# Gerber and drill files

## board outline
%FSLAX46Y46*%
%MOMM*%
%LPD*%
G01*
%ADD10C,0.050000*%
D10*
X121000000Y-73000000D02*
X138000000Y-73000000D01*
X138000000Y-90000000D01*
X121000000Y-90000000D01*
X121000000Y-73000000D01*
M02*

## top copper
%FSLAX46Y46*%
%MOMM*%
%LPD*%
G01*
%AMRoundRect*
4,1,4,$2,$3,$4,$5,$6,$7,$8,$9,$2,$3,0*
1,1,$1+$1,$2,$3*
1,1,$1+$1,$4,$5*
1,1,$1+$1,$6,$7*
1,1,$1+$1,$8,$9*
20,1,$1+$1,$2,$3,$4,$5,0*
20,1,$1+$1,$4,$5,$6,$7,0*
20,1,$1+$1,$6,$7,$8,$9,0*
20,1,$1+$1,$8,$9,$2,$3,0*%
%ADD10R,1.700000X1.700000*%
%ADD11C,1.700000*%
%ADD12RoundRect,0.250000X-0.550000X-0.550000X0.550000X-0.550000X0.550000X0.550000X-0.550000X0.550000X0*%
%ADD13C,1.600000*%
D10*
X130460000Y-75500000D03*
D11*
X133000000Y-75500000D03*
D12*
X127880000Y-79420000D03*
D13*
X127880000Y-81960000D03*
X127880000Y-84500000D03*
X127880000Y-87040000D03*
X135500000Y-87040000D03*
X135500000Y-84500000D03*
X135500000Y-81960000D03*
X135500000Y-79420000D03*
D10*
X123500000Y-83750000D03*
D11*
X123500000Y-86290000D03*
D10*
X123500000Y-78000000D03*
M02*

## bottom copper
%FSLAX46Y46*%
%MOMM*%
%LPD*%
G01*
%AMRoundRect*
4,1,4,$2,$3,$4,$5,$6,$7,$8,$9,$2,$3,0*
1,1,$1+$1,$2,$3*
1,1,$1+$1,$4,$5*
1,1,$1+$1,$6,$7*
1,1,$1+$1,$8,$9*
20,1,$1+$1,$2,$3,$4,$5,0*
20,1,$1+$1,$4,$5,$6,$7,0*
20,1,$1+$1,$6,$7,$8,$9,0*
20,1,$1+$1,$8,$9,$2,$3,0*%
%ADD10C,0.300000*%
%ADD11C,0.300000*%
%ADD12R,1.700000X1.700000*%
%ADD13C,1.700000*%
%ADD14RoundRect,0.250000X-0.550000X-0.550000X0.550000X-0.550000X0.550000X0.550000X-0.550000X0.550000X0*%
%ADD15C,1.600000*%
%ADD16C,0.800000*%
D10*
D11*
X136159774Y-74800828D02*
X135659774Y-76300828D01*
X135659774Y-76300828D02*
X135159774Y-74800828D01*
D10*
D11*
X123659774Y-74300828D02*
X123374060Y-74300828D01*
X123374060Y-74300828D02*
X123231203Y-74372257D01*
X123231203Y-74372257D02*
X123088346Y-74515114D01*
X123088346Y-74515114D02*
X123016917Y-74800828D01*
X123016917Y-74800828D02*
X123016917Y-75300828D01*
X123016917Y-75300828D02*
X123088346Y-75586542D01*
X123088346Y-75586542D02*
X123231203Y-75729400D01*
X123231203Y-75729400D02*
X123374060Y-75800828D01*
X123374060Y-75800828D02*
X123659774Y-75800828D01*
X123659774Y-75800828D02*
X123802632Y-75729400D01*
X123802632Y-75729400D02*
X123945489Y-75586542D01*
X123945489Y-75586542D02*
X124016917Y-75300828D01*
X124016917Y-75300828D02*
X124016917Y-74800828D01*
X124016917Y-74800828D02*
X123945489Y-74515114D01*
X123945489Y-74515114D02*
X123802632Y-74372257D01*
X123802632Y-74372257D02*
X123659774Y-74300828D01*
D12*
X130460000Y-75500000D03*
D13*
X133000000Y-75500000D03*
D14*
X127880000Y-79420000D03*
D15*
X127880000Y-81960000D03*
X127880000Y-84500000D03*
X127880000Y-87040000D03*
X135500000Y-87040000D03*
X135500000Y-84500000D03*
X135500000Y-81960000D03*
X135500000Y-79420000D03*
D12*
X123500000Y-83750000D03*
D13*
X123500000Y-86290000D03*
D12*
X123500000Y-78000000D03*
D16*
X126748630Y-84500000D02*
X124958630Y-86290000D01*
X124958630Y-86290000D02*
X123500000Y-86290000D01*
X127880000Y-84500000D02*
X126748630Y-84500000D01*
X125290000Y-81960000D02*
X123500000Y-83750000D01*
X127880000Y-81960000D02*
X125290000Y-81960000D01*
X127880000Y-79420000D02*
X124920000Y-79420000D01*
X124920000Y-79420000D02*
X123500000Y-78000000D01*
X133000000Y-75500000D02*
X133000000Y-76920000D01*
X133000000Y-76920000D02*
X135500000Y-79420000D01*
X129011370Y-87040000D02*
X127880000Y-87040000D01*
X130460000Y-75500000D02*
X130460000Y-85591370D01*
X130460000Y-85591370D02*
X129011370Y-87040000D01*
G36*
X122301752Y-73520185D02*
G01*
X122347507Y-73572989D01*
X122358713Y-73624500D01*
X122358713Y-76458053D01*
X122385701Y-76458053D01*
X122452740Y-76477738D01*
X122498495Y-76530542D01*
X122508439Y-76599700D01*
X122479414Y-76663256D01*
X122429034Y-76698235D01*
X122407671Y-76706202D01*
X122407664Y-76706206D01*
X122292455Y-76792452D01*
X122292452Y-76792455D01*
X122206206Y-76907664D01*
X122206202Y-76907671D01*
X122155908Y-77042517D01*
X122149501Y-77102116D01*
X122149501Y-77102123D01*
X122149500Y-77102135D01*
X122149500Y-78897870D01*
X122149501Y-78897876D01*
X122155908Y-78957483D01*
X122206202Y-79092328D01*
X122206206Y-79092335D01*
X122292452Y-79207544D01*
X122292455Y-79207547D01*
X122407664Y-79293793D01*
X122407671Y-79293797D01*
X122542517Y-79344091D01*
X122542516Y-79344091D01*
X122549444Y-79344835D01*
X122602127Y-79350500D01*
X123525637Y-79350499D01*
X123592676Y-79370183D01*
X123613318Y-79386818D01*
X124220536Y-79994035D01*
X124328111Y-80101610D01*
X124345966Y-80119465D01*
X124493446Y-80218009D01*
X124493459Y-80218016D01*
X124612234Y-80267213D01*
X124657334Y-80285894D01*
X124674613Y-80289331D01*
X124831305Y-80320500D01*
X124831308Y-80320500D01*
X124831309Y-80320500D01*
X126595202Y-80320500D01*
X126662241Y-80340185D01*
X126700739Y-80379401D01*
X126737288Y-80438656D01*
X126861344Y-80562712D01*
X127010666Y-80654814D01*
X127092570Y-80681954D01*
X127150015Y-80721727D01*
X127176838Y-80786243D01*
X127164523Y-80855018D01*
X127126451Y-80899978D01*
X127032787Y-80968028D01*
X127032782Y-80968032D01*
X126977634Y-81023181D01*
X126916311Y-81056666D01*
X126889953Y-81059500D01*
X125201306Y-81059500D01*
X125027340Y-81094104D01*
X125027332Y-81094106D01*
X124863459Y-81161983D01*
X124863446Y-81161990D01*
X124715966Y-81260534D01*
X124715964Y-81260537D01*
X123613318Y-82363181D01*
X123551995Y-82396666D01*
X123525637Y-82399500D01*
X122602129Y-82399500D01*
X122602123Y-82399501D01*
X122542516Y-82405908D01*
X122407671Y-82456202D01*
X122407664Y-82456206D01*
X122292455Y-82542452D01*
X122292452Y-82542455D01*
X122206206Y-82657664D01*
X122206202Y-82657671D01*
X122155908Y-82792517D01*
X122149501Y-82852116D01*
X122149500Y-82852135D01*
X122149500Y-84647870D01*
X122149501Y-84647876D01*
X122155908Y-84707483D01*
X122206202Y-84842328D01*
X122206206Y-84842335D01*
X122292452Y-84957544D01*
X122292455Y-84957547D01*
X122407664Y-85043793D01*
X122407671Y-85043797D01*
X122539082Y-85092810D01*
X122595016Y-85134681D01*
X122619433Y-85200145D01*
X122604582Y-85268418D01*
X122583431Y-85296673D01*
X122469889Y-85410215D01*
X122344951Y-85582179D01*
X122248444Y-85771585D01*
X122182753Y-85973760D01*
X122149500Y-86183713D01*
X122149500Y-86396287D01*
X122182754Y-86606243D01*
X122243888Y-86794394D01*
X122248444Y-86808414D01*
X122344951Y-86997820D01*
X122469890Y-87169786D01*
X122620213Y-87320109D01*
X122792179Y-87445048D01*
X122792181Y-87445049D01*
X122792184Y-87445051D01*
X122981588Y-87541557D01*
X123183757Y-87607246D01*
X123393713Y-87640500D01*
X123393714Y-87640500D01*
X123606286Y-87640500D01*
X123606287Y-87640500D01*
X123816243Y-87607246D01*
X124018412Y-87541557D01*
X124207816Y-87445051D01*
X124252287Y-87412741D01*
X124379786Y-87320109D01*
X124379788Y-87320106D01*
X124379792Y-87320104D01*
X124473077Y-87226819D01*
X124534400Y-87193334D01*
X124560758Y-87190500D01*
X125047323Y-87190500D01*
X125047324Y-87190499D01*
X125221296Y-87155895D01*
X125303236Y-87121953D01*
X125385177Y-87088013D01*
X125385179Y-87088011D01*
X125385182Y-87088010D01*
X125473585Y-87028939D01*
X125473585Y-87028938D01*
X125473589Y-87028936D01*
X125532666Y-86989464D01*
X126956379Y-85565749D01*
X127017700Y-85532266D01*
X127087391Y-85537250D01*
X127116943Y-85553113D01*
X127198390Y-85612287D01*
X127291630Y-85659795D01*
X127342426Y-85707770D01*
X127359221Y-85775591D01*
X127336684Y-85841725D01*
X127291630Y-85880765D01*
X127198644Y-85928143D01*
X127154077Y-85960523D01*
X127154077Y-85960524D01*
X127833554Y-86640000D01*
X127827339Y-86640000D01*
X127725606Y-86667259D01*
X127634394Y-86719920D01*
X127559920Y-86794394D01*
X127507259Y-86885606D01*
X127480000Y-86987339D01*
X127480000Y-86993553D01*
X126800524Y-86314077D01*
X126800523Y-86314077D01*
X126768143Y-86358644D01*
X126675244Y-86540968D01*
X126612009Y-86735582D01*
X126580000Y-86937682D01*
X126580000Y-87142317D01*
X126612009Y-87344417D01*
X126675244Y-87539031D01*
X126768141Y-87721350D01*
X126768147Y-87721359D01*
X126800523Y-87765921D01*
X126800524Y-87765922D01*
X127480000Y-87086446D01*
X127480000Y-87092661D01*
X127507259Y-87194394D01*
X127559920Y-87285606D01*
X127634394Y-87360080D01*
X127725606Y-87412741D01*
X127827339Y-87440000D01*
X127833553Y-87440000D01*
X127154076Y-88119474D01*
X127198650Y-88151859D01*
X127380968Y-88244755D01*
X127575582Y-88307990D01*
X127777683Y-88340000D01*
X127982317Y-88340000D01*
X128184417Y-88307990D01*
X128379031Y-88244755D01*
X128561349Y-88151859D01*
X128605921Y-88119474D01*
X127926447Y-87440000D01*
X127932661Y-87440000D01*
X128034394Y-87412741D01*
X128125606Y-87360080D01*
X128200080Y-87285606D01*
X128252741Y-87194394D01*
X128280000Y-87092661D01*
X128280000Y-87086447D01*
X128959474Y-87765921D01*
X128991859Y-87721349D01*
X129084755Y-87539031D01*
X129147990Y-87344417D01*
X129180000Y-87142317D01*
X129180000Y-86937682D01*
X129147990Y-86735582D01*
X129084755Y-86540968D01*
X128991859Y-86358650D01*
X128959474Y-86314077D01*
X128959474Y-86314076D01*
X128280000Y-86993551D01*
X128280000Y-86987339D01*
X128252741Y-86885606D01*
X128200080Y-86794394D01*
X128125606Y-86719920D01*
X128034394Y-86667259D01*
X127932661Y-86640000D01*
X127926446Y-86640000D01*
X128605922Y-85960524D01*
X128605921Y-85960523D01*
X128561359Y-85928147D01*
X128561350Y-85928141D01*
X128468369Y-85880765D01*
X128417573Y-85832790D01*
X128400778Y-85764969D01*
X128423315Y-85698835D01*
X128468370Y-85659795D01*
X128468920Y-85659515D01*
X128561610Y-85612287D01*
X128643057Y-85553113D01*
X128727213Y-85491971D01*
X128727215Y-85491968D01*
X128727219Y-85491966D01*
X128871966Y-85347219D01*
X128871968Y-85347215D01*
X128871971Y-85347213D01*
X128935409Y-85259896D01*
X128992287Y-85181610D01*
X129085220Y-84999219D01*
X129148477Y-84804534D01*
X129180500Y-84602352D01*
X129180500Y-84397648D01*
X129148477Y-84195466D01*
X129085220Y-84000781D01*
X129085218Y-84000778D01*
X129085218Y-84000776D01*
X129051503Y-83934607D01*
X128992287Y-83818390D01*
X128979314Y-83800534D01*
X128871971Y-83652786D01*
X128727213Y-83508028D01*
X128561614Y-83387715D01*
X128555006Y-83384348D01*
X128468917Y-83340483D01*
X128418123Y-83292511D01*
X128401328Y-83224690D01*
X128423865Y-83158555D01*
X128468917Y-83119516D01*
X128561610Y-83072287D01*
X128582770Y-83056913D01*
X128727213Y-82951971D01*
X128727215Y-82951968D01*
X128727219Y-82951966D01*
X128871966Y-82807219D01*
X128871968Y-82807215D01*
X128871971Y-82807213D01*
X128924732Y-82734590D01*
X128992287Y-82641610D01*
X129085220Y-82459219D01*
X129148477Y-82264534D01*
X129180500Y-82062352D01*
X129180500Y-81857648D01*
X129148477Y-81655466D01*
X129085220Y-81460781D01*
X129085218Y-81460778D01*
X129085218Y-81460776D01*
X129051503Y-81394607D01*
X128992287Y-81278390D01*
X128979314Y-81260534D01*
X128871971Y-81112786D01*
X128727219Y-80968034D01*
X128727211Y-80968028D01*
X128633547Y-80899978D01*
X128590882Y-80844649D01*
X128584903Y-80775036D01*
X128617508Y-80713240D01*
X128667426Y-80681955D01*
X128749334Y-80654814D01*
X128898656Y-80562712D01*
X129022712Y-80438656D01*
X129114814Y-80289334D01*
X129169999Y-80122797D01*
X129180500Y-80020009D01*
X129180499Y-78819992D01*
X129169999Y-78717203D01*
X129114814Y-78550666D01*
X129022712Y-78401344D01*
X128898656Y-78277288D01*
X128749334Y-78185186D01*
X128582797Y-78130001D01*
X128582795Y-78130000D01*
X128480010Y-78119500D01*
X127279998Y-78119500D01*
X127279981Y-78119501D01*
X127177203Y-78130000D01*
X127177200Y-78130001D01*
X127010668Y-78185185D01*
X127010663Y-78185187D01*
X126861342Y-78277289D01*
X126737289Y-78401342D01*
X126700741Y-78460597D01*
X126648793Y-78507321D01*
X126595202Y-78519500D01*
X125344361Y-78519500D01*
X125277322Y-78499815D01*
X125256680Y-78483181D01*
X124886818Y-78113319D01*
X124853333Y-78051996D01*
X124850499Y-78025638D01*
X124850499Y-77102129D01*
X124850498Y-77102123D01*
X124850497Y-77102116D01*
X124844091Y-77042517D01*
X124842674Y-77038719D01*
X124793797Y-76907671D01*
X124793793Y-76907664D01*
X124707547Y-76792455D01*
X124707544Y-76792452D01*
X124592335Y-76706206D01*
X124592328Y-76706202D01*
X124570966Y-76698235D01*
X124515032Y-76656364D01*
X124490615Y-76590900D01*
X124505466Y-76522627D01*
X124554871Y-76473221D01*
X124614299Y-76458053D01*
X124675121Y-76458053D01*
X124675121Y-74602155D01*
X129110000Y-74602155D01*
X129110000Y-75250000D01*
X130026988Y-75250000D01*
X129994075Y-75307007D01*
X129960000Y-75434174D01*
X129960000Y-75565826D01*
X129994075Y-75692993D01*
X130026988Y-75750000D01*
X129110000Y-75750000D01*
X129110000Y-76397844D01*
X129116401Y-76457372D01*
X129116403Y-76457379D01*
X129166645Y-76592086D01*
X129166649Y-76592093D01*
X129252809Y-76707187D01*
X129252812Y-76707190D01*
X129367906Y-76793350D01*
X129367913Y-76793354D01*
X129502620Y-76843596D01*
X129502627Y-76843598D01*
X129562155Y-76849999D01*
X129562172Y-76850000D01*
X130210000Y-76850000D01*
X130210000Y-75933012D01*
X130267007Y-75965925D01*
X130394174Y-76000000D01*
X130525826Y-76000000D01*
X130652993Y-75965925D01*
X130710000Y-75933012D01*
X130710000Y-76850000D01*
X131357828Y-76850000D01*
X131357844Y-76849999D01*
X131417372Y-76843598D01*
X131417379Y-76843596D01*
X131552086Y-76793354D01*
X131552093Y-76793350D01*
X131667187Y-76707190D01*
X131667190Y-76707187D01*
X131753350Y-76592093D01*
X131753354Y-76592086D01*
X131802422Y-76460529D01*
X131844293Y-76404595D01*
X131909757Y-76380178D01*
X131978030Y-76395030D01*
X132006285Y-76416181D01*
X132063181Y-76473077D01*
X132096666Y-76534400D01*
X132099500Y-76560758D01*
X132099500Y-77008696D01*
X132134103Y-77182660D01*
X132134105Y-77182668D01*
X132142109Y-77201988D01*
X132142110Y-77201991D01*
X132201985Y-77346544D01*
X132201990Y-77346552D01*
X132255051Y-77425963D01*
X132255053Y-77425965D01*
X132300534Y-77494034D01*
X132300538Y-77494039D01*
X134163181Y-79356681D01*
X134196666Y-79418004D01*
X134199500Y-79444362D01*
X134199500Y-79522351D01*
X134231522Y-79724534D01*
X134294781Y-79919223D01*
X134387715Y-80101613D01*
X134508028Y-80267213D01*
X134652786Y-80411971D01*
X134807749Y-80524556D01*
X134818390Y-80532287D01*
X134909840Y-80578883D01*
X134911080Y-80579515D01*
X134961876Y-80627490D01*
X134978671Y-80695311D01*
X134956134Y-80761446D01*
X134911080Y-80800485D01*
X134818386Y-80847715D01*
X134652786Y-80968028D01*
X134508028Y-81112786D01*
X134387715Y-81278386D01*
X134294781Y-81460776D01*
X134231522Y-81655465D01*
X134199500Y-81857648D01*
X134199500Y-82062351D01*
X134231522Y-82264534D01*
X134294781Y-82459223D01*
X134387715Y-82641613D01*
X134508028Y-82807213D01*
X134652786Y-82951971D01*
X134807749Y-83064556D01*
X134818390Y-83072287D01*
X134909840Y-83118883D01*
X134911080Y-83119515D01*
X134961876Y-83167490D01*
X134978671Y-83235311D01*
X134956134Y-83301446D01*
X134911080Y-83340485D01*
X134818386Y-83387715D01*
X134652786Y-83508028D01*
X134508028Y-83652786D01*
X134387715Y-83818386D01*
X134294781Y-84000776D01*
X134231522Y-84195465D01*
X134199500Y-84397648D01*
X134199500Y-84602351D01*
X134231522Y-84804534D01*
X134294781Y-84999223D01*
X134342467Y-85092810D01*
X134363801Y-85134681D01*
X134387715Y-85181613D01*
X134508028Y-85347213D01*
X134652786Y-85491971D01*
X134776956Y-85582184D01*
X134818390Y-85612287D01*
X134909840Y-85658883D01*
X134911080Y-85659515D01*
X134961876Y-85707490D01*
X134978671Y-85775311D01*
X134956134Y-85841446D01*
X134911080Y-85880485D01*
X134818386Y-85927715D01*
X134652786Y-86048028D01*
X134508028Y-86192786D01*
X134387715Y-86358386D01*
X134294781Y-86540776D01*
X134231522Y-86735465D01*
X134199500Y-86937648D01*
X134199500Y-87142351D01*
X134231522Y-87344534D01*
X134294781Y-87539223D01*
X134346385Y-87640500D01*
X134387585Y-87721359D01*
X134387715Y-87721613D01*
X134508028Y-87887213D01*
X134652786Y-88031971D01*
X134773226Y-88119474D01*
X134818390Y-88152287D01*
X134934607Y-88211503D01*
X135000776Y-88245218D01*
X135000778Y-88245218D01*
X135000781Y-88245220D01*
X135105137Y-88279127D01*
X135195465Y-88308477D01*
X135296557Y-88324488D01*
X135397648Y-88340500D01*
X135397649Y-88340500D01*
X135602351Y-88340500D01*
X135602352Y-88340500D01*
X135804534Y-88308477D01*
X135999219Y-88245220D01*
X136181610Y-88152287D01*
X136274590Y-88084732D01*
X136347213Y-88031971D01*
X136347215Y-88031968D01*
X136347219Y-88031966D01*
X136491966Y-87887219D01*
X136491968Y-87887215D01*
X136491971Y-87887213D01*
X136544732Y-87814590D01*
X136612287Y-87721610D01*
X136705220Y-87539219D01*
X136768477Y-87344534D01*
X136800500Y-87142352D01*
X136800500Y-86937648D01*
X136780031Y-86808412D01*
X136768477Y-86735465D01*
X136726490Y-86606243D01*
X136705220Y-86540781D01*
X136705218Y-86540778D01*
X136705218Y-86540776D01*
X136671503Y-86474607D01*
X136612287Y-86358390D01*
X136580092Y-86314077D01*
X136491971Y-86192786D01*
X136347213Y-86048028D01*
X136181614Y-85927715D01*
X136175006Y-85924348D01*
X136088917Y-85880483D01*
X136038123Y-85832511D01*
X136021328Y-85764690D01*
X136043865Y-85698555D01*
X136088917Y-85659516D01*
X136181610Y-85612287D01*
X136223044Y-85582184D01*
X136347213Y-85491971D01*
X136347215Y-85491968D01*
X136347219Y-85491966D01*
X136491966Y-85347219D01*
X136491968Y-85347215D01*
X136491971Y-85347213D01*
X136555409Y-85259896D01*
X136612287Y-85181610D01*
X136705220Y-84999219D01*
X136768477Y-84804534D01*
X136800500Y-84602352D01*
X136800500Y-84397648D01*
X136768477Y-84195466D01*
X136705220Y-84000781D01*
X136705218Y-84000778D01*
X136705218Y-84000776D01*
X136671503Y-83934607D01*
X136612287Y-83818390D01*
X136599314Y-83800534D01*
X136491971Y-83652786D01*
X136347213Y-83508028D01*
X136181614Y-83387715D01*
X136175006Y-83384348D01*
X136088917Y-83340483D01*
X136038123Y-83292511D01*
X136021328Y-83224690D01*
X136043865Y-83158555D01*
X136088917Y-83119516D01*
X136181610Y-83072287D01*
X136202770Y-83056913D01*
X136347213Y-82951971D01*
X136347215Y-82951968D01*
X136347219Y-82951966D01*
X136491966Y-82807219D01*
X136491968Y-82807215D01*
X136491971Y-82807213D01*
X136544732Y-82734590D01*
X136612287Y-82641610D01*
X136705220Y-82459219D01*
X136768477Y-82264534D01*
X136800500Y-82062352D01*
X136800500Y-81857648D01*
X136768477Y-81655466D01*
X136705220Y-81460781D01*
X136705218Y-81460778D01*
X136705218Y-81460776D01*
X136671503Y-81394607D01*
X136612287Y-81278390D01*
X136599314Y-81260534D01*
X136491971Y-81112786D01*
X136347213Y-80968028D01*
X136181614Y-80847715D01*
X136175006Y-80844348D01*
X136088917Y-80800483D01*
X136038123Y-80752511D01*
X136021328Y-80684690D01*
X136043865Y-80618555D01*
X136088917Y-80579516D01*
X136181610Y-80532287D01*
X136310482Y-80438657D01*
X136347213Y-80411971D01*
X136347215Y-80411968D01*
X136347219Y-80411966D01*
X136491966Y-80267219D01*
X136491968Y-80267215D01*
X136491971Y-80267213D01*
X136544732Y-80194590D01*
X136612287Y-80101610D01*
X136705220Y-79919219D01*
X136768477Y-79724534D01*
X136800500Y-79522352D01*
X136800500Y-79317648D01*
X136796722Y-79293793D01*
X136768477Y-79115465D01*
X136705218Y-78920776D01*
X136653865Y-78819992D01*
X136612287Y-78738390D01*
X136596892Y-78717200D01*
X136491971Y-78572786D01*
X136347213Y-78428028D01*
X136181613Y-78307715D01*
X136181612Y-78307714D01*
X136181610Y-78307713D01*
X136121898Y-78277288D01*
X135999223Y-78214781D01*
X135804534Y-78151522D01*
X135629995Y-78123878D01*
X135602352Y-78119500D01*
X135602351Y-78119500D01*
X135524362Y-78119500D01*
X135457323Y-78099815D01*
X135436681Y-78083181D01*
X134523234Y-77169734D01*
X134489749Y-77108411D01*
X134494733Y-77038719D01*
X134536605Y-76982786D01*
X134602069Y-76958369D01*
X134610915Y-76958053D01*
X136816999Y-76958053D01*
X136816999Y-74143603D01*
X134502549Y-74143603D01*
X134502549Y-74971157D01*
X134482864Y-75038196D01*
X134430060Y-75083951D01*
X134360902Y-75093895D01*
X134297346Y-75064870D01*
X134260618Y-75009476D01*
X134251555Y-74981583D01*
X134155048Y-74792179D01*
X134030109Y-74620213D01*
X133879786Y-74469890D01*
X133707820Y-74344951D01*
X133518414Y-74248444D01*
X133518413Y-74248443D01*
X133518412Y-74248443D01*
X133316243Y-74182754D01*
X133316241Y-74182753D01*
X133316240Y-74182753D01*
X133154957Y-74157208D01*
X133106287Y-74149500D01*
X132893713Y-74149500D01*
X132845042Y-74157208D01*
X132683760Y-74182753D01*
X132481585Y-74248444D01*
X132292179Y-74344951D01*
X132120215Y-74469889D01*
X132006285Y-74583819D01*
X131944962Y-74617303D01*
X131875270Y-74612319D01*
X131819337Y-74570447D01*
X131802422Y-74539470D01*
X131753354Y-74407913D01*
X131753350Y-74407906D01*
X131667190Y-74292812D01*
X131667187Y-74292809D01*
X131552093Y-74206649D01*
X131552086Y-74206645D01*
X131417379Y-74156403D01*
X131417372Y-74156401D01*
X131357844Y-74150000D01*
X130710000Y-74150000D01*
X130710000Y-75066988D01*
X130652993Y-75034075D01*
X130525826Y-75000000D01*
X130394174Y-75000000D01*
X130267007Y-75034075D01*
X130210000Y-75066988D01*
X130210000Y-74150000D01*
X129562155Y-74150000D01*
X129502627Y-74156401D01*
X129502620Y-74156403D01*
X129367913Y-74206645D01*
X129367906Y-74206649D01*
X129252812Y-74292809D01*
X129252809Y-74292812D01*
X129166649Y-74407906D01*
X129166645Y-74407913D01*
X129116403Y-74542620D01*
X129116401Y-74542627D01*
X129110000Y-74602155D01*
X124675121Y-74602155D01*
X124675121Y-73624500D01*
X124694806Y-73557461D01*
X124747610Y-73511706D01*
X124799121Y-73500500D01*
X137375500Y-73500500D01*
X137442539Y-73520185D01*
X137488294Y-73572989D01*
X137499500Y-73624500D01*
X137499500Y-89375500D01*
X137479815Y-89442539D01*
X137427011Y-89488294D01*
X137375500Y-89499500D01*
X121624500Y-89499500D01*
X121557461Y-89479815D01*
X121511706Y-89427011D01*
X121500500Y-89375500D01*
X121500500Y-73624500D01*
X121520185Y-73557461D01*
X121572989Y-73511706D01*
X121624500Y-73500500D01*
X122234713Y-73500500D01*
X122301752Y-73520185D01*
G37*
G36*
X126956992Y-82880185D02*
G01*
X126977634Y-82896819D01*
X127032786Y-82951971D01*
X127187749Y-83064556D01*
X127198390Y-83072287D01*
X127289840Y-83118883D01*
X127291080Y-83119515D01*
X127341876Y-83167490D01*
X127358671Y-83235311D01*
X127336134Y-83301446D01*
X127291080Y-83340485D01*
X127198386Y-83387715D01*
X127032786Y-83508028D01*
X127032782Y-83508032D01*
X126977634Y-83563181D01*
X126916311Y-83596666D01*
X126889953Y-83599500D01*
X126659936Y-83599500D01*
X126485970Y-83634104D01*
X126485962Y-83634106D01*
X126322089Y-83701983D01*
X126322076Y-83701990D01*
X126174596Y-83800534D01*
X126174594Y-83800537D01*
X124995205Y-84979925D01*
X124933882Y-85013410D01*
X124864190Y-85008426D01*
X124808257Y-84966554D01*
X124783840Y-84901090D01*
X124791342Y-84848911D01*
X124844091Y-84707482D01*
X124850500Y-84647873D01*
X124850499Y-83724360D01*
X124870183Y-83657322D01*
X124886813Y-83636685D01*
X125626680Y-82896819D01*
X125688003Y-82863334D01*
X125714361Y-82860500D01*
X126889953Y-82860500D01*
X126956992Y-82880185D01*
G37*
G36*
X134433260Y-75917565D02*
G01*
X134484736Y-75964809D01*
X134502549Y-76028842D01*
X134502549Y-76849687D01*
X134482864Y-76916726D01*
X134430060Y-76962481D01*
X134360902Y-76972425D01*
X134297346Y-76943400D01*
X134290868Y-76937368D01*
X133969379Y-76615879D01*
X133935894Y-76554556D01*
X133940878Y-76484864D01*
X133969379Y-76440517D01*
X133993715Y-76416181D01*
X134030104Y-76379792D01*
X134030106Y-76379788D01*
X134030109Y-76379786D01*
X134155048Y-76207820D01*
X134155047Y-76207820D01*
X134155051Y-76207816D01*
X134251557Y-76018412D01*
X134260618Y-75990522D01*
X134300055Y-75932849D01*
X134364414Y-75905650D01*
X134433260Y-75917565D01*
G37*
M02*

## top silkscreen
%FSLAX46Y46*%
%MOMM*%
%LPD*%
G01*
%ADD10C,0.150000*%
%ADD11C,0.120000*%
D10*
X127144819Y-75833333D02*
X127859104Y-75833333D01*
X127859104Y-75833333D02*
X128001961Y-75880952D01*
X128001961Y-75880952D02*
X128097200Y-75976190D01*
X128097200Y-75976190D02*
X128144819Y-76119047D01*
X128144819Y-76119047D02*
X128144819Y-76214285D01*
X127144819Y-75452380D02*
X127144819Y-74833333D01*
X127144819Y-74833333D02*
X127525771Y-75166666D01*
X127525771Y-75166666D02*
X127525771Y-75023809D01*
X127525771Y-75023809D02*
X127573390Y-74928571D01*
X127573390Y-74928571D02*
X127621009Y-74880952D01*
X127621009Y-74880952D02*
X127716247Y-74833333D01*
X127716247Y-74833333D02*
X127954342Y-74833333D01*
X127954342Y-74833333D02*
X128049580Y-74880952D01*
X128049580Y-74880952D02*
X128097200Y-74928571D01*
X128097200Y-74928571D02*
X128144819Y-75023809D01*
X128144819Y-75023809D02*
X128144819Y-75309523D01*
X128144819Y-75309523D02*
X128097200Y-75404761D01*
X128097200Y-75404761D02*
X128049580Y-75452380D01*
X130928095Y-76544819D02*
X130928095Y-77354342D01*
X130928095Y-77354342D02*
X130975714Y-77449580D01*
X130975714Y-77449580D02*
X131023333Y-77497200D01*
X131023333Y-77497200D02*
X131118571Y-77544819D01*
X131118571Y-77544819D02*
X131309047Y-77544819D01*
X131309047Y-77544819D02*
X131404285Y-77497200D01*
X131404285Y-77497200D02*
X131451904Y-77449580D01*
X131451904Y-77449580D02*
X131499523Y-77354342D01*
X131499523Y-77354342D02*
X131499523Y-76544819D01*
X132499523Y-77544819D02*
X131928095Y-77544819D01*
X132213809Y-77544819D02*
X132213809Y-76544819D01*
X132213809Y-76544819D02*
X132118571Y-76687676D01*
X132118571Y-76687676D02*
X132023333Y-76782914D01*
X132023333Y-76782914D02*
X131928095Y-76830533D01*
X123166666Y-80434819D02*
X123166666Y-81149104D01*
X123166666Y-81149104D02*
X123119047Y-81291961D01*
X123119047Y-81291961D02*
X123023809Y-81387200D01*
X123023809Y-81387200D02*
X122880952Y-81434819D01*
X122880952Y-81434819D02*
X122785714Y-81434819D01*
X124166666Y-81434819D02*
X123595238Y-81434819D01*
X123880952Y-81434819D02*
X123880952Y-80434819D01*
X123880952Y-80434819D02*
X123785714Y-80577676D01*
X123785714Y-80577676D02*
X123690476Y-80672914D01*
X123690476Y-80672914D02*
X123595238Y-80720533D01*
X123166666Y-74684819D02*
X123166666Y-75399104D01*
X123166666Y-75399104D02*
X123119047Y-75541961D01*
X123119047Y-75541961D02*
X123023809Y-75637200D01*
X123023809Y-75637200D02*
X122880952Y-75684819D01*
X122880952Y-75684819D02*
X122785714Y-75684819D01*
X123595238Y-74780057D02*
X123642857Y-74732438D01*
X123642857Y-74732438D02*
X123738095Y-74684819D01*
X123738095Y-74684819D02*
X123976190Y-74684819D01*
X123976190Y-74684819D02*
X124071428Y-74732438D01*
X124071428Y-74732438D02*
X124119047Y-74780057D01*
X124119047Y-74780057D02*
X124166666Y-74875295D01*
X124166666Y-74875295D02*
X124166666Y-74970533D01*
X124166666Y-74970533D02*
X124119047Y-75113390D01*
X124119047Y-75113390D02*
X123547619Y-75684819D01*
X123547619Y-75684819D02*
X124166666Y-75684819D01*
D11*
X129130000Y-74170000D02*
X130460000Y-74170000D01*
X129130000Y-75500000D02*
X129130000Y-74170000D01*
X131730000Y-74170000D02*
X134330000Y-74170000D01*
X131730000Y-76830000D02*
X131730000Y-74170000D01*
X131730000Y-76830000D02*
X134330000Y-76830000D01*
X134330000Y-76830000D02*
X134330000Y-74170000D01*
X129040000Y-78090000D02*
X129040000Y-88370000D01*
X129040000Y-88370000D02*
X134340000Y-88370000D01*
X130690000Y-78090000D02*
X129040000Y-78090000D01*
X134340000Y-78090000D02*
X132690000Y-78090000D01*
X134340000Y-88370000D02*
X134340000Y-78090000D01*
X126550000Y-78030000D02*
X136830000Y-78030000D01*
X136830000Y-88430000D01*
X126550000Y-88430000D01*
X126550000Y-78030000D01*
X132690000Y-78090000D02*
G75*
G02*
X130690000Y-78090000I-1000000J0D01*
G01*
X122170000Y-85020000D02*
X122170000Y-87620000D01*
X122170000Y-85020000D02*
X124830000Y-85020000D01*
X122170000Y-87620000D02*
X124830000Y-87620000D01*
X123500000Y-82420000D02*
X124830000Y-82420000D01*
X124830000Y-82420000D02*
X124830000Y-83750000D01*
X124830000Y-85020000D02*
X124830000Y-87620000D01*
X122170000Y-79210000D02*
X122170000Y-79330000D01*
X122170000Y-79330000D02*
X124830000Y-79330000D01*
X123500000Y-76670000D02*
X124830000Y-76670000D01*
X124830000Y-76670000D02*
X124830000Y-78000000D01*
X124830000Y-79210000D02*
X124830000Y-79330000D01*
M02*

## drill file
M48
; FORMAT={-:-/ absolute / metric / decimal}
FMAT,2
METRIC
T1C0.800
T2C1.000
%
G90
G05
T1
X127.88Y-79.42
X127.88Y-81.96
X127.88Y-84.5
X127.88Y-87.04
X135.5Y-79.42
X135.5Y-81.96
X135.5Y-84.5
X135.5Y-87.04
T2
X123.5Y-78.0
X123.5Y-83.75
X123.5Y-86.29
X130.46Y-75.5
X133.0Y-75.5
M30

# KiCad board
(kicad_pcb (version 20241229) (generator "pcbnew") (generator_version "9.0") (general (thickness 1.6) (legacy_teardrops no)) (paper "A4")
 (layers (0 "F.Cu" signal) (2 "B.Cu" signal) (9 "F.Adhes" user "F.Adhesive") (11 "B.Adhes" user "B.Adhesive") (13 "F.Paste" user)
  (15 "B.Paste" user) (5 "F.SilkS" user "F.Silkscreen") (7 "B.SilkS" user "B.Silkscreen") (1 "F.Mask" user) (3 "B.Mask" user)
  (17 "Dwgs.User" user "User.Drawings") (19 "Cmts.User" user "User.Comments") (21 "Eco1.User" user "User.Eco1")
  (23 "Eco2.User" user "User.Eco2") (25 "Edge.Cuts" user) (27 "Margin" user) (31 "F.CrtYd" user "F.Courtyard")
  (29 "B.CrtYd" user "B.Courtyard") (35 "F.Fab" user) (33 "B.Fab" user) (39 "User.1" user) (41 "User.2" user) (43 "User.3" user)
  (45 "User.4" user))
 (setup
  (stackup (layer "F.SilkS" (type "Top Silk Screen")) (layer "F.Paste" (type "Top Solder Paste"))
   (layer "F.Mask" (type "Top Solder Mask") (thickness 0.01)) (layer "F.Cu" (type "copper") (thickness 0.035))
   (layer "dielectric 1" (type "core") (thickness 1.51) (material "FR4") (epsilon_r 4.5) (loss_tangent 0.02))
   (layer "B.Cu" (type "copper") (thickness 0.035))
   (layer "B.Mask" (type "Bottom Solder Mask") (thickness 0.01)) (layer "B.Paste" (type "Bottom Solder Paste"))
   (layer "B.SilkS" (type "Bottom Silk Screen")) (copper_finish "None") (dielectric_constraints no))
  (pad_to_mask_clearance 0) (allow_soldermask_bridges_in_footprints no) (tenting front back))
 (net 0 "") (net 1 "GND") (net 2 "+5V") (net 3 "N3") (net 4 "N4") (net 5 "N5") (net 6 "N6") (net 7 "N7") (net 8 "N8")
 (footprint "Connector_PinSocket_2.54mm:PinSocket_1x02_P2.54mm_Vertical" (layer "F.Cu") (at 130.46 75.5 90)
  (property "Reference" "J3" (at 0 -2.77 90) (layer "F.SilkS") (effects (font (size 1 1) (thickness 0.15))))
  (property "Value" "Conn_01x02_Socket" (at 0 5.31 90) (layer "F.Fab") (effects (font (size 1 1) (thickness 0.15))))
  (fp_line (start 1.33 -1.33) (end 1.33 0) (stroke (width 0.12) (type solid)) (layer "F.SilkS"))
  (fp_line (start 0 -1.33) (end 1.33 -1.33) (stroke (width 0.12) (type solid)) (layer "F.SilkS"))
  (fp_line (start 1.33 1.27) (end 1.33 3.87) (stroke (width 0.12) (type solid)) (layer "F.SilkS"))
  (fp_line (start -1.33 1.27) (end 1.33 1.27) (stroke (width 0.12) (type solid)) (layer "F.SilkS"))
  (fp_line (start -1.33 1.27) (end -1.33 3.87) (stroke (width 0.12) (type solid)) (layer "F.SilkS"))
  (fp_line (start -1.33 3.87) (end 1.33 3.87) (stroke (width 0.12) (type solid)) (layer "F.SilkS"))
  (pad "1" thru_hole rect (at 0 0 90) (size 1.7 1.7) (drill 1) (layers "*.Cu" "*.Mask") (remove_unused_layers no) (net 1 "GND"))
  (pad "2" thru_hole circle (at 0 2.54 90) (size 1.7 1.7) (drill 1) (layers "*.Cu" "*.Mask") (remove_unused_layers no) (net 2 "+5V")))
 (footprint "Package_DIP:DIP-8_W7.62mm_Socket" (layer "F.Cu") (at 127.88 79.42)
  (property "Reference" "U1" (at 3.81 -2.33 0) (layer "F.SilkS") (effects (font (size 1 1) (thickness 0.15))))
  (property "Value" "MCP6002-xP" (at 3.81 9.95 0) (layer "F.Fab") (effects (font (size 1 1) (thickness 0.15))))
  (fp_line (start 1.16 -1.33) (end 1.16 8.95) (stroke (width 0.12) (type solid)) (layer "F.SilkS"))
  (fp_line (start 1.16 8.95) (end 6.46 8.95) (stroke (width 0.12) (type solid)) (layer "F.SilkS"))
  (fp_line (start 2.81 -1.33) (end 1.16 -1.33) (stroke (width 0.12) (type solid)) (layer "F.SilkS"))
  (fp_line (start 6.46 -1.33) (end 4.81 -1.33) (stroke (width 0.12) (type solid)) (layer "F.SilkS"))
  (fp_line (start 6.46 8.95) (end 6.46 -1.33) (stroke (width 0.12) (type solid)) (layer "F.SilkS"))
  (fp_rect (start -1.33 -1.39) (end 8.95 9.01) (stroke (width 0.12) (type solid)) (fill no) (layer "F.SilkS"))
  (fp_arc (start 4.81 -1.33) (mid 3.81 -0.33) (end 2.81 -1.33) (stroke (width 0.12) (type solid)) (layer "F.SilkS"))
  (pad "1" thru_hole roundrect (at 0 0) (size 1.6 1.6) (drill 0.8) (layers "*.Cu" "*.Mask") (remove_unused_layers no)
   (roundrect_rratio 0.15625) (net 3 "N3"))
  (pad "2" thru_hole circle (at 0 2.54) (size 1.6 1.6) (drill 0.8) (layers "*.Cu" "*.Mask") (remove_unused_layers no) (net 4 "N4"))
  (pad "3" thru_hole circle (at 0 5.08) (size 1.6 1.6) (drill 0.8) (layers "*.Cu" "*.Mask") (remove_unused_layers no) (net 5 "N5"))
  (pad "4" thru_hole circle (at 0 7.62) (size 1.6 1.6) (drill 0.8) (layers "*.Cu" "*.Mask") (remove_unused_layers no) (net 1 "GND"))
  (pad "5" thru_hole circle (at 7.62 7.62) (size 1.6 1.6) (drill 0.8) (layers "*.Cu" "*.Mask") (remove_unused_layers no) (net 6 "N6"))
  (pad "6" thru_hole circle (at 7.62 5.08) (size 1.6 1.6) (drill 0.8) (layers "*.Cu" "*.Mask") (remove_unused_layers no) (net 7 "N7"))
  (pad "7" thru_hole circle (at 7.62 2.54) (size 1.6 1.6) (drill 0.8) (layers "*.Cu" "*.Mask") (remove_unused_layers no) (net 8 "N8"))
  (pad "8" thru_hole circle (at 7.62 0) (size 1.6 1.6) (drill 0.8) (layers "*.Cu" "*.Mask") (remove_unused_layers no) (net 2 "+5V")))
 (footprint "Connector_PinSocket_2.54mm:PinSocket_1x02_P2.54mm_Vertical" (layer "F.Cu") (at 123.5 83.75)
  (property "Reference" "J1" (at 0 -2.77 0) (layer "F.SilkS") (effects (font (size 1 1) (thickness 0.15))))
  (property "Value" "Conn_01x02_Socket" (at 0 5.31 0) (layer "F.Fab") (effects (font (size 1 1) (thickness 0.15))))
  (fp_line (start -1.33 1.27) (end -1.33 3.87) (stroke (width 0.12) (type solid)) (layer "F.SilkS"))
  (fp_line (start -1.33 1.27) (end 1.33 1.27) (stroke (width 0.12) (type solid)) (layer "F.SilkS"))
  (fp_line (start -1.33 3.87) (end 1.33 3.87) (stroke (width 0.12) (type solid)) (layer "F.SilkS"))
  (fp_line (start 0 -1.33) (end 1.33 -1.33) (stroke (width 0.12) (type solid)) (layer "F.SilkS"))
  (fp_line (start 1.33 -1.33) (end 1.33 0) (stroke (width 0.12) (type solid)) (layer "F.SilkS"))
  (fp_line (start 1.33 1.27) (end 1.33 3.87) (stroke (width 0.12) (type solid)) (layer "F.SilkS"))
  (pad "1" thru_hole rect (at 0 0) (size 1.7 1.7) (drill 1) (layers "*.Cu" "*.Mask") (remove_unused_layers no) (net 4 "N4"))
  (pad "2" thru_hole circle (at 0 2.54) (size 1.7 1.7) (drill 1) (layers "*.Cu" "*.Mask") (remove_unused_layers no) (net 5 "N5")))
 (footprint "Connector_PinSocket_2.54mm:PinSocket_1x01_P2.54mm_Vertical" (layer "F.Cu") (at 123.5 78)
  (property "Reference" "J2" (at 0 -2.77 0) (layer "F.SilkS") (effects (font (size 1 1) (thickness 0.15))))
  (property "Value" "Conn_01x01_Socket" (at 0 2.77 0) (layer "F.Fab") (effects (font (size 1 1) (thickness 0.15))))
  (fp_line (start -1.33 1.21) (end -1.33 1.33) (stroke (width 0.12) (type solid)) (layer "F.SilkS"))
  (fp_line (start -1.33 1.33) (end 1.33 1.33) (stroke (width 0.12) (type solid)) (layer "F.SilkS"))
  (fp_line (start 0 -1.33) (end 1.33 -1.33) (stroke (width 0.12) (type solid)) (layer "F.SilkS"))
  (fp_line (start 1.33 -1.33) (end 1.33 0) (stroke (width 0.12) (type solid)) (layer "F.SilkS"))
  (fp_line (start 1.33 1.21) (end 1.33 1.33) (stroke (width 0.12) (type solid)) (layer "F.SilkS"))
  (pad "1" thru_hole rect (at 0 0) (size 1.7 1.7) (drill 1) (layers "*.Cu" "*.Mask") (remove_unused_layers no) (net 3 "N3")))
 (gr_rect (start 121 73) (end 138 90) (stroke (width 0.05) (type default)) (fill no) (layer "Edge.Cuts"))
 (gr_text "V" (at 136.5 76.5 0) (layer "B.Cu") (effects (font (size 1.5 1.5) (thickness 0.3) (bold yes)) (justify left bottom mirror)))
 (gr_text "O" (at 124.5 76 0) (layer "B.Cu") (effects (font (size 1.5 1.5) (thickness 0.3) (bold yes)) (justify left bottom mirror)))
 (segment (start 126.74863 84.5) (end 124.95863 86.29) (width 0.8) (layer "B.Cu") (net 5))
 (segment (start 124.95863 86.29) (end 123.5 86.29) (width 0.8) (layer "B.Cu") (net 5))
 (segment (start 127.88 84.5) (end 126.74863 84.5) (width 0.8) (layer "B.Cu") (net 5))
 (segment (start 125.29 81.96) (end 123.5 83.75) (width 0.8) (layer "B.Cu") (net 4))
 (segment (start 127.88 81.96) (end 125.29 81.96) (width 0.8) (layer "B.Cu") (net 4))
 (segment (start 127.88 79.42) (end 124.92 79.42) (width 0.8) (layer "B.Cu") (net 3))
 (segment (start 124.92 79.42) (end 123.5 78) (width 0.8) (layer "B.Cu") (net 3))
 (segment (start 133 75.5) (end 133 76.92) (width 0.8) (layer "B.Cu") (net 2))
 (segment (start 133 76.92) (end 135.5 79.42) (width 0.8) (layer "B.Cu") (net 2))
 (segment (start 129.01137 87.04) (end 127.88 87.04) (width 0.8) (layer "B.Cu") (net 1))
 (segment (start 130.46 75.5) (end 130.46 85.59137) (width 0.8) (layer "B.Cu") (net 1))
 (segment (start 130.46 85.59137) (end 129.01137 87.04) (width 0.8) (layer "B.Cu") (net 1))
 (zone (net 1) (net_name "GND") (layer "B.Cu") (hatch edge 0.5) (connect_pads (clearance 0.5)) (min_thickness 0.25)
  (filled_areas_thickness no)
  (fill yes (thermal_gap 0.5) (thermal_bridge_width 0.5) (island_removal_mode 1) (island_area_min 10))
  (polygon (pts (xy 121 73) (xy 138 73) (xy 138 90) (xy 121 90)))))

